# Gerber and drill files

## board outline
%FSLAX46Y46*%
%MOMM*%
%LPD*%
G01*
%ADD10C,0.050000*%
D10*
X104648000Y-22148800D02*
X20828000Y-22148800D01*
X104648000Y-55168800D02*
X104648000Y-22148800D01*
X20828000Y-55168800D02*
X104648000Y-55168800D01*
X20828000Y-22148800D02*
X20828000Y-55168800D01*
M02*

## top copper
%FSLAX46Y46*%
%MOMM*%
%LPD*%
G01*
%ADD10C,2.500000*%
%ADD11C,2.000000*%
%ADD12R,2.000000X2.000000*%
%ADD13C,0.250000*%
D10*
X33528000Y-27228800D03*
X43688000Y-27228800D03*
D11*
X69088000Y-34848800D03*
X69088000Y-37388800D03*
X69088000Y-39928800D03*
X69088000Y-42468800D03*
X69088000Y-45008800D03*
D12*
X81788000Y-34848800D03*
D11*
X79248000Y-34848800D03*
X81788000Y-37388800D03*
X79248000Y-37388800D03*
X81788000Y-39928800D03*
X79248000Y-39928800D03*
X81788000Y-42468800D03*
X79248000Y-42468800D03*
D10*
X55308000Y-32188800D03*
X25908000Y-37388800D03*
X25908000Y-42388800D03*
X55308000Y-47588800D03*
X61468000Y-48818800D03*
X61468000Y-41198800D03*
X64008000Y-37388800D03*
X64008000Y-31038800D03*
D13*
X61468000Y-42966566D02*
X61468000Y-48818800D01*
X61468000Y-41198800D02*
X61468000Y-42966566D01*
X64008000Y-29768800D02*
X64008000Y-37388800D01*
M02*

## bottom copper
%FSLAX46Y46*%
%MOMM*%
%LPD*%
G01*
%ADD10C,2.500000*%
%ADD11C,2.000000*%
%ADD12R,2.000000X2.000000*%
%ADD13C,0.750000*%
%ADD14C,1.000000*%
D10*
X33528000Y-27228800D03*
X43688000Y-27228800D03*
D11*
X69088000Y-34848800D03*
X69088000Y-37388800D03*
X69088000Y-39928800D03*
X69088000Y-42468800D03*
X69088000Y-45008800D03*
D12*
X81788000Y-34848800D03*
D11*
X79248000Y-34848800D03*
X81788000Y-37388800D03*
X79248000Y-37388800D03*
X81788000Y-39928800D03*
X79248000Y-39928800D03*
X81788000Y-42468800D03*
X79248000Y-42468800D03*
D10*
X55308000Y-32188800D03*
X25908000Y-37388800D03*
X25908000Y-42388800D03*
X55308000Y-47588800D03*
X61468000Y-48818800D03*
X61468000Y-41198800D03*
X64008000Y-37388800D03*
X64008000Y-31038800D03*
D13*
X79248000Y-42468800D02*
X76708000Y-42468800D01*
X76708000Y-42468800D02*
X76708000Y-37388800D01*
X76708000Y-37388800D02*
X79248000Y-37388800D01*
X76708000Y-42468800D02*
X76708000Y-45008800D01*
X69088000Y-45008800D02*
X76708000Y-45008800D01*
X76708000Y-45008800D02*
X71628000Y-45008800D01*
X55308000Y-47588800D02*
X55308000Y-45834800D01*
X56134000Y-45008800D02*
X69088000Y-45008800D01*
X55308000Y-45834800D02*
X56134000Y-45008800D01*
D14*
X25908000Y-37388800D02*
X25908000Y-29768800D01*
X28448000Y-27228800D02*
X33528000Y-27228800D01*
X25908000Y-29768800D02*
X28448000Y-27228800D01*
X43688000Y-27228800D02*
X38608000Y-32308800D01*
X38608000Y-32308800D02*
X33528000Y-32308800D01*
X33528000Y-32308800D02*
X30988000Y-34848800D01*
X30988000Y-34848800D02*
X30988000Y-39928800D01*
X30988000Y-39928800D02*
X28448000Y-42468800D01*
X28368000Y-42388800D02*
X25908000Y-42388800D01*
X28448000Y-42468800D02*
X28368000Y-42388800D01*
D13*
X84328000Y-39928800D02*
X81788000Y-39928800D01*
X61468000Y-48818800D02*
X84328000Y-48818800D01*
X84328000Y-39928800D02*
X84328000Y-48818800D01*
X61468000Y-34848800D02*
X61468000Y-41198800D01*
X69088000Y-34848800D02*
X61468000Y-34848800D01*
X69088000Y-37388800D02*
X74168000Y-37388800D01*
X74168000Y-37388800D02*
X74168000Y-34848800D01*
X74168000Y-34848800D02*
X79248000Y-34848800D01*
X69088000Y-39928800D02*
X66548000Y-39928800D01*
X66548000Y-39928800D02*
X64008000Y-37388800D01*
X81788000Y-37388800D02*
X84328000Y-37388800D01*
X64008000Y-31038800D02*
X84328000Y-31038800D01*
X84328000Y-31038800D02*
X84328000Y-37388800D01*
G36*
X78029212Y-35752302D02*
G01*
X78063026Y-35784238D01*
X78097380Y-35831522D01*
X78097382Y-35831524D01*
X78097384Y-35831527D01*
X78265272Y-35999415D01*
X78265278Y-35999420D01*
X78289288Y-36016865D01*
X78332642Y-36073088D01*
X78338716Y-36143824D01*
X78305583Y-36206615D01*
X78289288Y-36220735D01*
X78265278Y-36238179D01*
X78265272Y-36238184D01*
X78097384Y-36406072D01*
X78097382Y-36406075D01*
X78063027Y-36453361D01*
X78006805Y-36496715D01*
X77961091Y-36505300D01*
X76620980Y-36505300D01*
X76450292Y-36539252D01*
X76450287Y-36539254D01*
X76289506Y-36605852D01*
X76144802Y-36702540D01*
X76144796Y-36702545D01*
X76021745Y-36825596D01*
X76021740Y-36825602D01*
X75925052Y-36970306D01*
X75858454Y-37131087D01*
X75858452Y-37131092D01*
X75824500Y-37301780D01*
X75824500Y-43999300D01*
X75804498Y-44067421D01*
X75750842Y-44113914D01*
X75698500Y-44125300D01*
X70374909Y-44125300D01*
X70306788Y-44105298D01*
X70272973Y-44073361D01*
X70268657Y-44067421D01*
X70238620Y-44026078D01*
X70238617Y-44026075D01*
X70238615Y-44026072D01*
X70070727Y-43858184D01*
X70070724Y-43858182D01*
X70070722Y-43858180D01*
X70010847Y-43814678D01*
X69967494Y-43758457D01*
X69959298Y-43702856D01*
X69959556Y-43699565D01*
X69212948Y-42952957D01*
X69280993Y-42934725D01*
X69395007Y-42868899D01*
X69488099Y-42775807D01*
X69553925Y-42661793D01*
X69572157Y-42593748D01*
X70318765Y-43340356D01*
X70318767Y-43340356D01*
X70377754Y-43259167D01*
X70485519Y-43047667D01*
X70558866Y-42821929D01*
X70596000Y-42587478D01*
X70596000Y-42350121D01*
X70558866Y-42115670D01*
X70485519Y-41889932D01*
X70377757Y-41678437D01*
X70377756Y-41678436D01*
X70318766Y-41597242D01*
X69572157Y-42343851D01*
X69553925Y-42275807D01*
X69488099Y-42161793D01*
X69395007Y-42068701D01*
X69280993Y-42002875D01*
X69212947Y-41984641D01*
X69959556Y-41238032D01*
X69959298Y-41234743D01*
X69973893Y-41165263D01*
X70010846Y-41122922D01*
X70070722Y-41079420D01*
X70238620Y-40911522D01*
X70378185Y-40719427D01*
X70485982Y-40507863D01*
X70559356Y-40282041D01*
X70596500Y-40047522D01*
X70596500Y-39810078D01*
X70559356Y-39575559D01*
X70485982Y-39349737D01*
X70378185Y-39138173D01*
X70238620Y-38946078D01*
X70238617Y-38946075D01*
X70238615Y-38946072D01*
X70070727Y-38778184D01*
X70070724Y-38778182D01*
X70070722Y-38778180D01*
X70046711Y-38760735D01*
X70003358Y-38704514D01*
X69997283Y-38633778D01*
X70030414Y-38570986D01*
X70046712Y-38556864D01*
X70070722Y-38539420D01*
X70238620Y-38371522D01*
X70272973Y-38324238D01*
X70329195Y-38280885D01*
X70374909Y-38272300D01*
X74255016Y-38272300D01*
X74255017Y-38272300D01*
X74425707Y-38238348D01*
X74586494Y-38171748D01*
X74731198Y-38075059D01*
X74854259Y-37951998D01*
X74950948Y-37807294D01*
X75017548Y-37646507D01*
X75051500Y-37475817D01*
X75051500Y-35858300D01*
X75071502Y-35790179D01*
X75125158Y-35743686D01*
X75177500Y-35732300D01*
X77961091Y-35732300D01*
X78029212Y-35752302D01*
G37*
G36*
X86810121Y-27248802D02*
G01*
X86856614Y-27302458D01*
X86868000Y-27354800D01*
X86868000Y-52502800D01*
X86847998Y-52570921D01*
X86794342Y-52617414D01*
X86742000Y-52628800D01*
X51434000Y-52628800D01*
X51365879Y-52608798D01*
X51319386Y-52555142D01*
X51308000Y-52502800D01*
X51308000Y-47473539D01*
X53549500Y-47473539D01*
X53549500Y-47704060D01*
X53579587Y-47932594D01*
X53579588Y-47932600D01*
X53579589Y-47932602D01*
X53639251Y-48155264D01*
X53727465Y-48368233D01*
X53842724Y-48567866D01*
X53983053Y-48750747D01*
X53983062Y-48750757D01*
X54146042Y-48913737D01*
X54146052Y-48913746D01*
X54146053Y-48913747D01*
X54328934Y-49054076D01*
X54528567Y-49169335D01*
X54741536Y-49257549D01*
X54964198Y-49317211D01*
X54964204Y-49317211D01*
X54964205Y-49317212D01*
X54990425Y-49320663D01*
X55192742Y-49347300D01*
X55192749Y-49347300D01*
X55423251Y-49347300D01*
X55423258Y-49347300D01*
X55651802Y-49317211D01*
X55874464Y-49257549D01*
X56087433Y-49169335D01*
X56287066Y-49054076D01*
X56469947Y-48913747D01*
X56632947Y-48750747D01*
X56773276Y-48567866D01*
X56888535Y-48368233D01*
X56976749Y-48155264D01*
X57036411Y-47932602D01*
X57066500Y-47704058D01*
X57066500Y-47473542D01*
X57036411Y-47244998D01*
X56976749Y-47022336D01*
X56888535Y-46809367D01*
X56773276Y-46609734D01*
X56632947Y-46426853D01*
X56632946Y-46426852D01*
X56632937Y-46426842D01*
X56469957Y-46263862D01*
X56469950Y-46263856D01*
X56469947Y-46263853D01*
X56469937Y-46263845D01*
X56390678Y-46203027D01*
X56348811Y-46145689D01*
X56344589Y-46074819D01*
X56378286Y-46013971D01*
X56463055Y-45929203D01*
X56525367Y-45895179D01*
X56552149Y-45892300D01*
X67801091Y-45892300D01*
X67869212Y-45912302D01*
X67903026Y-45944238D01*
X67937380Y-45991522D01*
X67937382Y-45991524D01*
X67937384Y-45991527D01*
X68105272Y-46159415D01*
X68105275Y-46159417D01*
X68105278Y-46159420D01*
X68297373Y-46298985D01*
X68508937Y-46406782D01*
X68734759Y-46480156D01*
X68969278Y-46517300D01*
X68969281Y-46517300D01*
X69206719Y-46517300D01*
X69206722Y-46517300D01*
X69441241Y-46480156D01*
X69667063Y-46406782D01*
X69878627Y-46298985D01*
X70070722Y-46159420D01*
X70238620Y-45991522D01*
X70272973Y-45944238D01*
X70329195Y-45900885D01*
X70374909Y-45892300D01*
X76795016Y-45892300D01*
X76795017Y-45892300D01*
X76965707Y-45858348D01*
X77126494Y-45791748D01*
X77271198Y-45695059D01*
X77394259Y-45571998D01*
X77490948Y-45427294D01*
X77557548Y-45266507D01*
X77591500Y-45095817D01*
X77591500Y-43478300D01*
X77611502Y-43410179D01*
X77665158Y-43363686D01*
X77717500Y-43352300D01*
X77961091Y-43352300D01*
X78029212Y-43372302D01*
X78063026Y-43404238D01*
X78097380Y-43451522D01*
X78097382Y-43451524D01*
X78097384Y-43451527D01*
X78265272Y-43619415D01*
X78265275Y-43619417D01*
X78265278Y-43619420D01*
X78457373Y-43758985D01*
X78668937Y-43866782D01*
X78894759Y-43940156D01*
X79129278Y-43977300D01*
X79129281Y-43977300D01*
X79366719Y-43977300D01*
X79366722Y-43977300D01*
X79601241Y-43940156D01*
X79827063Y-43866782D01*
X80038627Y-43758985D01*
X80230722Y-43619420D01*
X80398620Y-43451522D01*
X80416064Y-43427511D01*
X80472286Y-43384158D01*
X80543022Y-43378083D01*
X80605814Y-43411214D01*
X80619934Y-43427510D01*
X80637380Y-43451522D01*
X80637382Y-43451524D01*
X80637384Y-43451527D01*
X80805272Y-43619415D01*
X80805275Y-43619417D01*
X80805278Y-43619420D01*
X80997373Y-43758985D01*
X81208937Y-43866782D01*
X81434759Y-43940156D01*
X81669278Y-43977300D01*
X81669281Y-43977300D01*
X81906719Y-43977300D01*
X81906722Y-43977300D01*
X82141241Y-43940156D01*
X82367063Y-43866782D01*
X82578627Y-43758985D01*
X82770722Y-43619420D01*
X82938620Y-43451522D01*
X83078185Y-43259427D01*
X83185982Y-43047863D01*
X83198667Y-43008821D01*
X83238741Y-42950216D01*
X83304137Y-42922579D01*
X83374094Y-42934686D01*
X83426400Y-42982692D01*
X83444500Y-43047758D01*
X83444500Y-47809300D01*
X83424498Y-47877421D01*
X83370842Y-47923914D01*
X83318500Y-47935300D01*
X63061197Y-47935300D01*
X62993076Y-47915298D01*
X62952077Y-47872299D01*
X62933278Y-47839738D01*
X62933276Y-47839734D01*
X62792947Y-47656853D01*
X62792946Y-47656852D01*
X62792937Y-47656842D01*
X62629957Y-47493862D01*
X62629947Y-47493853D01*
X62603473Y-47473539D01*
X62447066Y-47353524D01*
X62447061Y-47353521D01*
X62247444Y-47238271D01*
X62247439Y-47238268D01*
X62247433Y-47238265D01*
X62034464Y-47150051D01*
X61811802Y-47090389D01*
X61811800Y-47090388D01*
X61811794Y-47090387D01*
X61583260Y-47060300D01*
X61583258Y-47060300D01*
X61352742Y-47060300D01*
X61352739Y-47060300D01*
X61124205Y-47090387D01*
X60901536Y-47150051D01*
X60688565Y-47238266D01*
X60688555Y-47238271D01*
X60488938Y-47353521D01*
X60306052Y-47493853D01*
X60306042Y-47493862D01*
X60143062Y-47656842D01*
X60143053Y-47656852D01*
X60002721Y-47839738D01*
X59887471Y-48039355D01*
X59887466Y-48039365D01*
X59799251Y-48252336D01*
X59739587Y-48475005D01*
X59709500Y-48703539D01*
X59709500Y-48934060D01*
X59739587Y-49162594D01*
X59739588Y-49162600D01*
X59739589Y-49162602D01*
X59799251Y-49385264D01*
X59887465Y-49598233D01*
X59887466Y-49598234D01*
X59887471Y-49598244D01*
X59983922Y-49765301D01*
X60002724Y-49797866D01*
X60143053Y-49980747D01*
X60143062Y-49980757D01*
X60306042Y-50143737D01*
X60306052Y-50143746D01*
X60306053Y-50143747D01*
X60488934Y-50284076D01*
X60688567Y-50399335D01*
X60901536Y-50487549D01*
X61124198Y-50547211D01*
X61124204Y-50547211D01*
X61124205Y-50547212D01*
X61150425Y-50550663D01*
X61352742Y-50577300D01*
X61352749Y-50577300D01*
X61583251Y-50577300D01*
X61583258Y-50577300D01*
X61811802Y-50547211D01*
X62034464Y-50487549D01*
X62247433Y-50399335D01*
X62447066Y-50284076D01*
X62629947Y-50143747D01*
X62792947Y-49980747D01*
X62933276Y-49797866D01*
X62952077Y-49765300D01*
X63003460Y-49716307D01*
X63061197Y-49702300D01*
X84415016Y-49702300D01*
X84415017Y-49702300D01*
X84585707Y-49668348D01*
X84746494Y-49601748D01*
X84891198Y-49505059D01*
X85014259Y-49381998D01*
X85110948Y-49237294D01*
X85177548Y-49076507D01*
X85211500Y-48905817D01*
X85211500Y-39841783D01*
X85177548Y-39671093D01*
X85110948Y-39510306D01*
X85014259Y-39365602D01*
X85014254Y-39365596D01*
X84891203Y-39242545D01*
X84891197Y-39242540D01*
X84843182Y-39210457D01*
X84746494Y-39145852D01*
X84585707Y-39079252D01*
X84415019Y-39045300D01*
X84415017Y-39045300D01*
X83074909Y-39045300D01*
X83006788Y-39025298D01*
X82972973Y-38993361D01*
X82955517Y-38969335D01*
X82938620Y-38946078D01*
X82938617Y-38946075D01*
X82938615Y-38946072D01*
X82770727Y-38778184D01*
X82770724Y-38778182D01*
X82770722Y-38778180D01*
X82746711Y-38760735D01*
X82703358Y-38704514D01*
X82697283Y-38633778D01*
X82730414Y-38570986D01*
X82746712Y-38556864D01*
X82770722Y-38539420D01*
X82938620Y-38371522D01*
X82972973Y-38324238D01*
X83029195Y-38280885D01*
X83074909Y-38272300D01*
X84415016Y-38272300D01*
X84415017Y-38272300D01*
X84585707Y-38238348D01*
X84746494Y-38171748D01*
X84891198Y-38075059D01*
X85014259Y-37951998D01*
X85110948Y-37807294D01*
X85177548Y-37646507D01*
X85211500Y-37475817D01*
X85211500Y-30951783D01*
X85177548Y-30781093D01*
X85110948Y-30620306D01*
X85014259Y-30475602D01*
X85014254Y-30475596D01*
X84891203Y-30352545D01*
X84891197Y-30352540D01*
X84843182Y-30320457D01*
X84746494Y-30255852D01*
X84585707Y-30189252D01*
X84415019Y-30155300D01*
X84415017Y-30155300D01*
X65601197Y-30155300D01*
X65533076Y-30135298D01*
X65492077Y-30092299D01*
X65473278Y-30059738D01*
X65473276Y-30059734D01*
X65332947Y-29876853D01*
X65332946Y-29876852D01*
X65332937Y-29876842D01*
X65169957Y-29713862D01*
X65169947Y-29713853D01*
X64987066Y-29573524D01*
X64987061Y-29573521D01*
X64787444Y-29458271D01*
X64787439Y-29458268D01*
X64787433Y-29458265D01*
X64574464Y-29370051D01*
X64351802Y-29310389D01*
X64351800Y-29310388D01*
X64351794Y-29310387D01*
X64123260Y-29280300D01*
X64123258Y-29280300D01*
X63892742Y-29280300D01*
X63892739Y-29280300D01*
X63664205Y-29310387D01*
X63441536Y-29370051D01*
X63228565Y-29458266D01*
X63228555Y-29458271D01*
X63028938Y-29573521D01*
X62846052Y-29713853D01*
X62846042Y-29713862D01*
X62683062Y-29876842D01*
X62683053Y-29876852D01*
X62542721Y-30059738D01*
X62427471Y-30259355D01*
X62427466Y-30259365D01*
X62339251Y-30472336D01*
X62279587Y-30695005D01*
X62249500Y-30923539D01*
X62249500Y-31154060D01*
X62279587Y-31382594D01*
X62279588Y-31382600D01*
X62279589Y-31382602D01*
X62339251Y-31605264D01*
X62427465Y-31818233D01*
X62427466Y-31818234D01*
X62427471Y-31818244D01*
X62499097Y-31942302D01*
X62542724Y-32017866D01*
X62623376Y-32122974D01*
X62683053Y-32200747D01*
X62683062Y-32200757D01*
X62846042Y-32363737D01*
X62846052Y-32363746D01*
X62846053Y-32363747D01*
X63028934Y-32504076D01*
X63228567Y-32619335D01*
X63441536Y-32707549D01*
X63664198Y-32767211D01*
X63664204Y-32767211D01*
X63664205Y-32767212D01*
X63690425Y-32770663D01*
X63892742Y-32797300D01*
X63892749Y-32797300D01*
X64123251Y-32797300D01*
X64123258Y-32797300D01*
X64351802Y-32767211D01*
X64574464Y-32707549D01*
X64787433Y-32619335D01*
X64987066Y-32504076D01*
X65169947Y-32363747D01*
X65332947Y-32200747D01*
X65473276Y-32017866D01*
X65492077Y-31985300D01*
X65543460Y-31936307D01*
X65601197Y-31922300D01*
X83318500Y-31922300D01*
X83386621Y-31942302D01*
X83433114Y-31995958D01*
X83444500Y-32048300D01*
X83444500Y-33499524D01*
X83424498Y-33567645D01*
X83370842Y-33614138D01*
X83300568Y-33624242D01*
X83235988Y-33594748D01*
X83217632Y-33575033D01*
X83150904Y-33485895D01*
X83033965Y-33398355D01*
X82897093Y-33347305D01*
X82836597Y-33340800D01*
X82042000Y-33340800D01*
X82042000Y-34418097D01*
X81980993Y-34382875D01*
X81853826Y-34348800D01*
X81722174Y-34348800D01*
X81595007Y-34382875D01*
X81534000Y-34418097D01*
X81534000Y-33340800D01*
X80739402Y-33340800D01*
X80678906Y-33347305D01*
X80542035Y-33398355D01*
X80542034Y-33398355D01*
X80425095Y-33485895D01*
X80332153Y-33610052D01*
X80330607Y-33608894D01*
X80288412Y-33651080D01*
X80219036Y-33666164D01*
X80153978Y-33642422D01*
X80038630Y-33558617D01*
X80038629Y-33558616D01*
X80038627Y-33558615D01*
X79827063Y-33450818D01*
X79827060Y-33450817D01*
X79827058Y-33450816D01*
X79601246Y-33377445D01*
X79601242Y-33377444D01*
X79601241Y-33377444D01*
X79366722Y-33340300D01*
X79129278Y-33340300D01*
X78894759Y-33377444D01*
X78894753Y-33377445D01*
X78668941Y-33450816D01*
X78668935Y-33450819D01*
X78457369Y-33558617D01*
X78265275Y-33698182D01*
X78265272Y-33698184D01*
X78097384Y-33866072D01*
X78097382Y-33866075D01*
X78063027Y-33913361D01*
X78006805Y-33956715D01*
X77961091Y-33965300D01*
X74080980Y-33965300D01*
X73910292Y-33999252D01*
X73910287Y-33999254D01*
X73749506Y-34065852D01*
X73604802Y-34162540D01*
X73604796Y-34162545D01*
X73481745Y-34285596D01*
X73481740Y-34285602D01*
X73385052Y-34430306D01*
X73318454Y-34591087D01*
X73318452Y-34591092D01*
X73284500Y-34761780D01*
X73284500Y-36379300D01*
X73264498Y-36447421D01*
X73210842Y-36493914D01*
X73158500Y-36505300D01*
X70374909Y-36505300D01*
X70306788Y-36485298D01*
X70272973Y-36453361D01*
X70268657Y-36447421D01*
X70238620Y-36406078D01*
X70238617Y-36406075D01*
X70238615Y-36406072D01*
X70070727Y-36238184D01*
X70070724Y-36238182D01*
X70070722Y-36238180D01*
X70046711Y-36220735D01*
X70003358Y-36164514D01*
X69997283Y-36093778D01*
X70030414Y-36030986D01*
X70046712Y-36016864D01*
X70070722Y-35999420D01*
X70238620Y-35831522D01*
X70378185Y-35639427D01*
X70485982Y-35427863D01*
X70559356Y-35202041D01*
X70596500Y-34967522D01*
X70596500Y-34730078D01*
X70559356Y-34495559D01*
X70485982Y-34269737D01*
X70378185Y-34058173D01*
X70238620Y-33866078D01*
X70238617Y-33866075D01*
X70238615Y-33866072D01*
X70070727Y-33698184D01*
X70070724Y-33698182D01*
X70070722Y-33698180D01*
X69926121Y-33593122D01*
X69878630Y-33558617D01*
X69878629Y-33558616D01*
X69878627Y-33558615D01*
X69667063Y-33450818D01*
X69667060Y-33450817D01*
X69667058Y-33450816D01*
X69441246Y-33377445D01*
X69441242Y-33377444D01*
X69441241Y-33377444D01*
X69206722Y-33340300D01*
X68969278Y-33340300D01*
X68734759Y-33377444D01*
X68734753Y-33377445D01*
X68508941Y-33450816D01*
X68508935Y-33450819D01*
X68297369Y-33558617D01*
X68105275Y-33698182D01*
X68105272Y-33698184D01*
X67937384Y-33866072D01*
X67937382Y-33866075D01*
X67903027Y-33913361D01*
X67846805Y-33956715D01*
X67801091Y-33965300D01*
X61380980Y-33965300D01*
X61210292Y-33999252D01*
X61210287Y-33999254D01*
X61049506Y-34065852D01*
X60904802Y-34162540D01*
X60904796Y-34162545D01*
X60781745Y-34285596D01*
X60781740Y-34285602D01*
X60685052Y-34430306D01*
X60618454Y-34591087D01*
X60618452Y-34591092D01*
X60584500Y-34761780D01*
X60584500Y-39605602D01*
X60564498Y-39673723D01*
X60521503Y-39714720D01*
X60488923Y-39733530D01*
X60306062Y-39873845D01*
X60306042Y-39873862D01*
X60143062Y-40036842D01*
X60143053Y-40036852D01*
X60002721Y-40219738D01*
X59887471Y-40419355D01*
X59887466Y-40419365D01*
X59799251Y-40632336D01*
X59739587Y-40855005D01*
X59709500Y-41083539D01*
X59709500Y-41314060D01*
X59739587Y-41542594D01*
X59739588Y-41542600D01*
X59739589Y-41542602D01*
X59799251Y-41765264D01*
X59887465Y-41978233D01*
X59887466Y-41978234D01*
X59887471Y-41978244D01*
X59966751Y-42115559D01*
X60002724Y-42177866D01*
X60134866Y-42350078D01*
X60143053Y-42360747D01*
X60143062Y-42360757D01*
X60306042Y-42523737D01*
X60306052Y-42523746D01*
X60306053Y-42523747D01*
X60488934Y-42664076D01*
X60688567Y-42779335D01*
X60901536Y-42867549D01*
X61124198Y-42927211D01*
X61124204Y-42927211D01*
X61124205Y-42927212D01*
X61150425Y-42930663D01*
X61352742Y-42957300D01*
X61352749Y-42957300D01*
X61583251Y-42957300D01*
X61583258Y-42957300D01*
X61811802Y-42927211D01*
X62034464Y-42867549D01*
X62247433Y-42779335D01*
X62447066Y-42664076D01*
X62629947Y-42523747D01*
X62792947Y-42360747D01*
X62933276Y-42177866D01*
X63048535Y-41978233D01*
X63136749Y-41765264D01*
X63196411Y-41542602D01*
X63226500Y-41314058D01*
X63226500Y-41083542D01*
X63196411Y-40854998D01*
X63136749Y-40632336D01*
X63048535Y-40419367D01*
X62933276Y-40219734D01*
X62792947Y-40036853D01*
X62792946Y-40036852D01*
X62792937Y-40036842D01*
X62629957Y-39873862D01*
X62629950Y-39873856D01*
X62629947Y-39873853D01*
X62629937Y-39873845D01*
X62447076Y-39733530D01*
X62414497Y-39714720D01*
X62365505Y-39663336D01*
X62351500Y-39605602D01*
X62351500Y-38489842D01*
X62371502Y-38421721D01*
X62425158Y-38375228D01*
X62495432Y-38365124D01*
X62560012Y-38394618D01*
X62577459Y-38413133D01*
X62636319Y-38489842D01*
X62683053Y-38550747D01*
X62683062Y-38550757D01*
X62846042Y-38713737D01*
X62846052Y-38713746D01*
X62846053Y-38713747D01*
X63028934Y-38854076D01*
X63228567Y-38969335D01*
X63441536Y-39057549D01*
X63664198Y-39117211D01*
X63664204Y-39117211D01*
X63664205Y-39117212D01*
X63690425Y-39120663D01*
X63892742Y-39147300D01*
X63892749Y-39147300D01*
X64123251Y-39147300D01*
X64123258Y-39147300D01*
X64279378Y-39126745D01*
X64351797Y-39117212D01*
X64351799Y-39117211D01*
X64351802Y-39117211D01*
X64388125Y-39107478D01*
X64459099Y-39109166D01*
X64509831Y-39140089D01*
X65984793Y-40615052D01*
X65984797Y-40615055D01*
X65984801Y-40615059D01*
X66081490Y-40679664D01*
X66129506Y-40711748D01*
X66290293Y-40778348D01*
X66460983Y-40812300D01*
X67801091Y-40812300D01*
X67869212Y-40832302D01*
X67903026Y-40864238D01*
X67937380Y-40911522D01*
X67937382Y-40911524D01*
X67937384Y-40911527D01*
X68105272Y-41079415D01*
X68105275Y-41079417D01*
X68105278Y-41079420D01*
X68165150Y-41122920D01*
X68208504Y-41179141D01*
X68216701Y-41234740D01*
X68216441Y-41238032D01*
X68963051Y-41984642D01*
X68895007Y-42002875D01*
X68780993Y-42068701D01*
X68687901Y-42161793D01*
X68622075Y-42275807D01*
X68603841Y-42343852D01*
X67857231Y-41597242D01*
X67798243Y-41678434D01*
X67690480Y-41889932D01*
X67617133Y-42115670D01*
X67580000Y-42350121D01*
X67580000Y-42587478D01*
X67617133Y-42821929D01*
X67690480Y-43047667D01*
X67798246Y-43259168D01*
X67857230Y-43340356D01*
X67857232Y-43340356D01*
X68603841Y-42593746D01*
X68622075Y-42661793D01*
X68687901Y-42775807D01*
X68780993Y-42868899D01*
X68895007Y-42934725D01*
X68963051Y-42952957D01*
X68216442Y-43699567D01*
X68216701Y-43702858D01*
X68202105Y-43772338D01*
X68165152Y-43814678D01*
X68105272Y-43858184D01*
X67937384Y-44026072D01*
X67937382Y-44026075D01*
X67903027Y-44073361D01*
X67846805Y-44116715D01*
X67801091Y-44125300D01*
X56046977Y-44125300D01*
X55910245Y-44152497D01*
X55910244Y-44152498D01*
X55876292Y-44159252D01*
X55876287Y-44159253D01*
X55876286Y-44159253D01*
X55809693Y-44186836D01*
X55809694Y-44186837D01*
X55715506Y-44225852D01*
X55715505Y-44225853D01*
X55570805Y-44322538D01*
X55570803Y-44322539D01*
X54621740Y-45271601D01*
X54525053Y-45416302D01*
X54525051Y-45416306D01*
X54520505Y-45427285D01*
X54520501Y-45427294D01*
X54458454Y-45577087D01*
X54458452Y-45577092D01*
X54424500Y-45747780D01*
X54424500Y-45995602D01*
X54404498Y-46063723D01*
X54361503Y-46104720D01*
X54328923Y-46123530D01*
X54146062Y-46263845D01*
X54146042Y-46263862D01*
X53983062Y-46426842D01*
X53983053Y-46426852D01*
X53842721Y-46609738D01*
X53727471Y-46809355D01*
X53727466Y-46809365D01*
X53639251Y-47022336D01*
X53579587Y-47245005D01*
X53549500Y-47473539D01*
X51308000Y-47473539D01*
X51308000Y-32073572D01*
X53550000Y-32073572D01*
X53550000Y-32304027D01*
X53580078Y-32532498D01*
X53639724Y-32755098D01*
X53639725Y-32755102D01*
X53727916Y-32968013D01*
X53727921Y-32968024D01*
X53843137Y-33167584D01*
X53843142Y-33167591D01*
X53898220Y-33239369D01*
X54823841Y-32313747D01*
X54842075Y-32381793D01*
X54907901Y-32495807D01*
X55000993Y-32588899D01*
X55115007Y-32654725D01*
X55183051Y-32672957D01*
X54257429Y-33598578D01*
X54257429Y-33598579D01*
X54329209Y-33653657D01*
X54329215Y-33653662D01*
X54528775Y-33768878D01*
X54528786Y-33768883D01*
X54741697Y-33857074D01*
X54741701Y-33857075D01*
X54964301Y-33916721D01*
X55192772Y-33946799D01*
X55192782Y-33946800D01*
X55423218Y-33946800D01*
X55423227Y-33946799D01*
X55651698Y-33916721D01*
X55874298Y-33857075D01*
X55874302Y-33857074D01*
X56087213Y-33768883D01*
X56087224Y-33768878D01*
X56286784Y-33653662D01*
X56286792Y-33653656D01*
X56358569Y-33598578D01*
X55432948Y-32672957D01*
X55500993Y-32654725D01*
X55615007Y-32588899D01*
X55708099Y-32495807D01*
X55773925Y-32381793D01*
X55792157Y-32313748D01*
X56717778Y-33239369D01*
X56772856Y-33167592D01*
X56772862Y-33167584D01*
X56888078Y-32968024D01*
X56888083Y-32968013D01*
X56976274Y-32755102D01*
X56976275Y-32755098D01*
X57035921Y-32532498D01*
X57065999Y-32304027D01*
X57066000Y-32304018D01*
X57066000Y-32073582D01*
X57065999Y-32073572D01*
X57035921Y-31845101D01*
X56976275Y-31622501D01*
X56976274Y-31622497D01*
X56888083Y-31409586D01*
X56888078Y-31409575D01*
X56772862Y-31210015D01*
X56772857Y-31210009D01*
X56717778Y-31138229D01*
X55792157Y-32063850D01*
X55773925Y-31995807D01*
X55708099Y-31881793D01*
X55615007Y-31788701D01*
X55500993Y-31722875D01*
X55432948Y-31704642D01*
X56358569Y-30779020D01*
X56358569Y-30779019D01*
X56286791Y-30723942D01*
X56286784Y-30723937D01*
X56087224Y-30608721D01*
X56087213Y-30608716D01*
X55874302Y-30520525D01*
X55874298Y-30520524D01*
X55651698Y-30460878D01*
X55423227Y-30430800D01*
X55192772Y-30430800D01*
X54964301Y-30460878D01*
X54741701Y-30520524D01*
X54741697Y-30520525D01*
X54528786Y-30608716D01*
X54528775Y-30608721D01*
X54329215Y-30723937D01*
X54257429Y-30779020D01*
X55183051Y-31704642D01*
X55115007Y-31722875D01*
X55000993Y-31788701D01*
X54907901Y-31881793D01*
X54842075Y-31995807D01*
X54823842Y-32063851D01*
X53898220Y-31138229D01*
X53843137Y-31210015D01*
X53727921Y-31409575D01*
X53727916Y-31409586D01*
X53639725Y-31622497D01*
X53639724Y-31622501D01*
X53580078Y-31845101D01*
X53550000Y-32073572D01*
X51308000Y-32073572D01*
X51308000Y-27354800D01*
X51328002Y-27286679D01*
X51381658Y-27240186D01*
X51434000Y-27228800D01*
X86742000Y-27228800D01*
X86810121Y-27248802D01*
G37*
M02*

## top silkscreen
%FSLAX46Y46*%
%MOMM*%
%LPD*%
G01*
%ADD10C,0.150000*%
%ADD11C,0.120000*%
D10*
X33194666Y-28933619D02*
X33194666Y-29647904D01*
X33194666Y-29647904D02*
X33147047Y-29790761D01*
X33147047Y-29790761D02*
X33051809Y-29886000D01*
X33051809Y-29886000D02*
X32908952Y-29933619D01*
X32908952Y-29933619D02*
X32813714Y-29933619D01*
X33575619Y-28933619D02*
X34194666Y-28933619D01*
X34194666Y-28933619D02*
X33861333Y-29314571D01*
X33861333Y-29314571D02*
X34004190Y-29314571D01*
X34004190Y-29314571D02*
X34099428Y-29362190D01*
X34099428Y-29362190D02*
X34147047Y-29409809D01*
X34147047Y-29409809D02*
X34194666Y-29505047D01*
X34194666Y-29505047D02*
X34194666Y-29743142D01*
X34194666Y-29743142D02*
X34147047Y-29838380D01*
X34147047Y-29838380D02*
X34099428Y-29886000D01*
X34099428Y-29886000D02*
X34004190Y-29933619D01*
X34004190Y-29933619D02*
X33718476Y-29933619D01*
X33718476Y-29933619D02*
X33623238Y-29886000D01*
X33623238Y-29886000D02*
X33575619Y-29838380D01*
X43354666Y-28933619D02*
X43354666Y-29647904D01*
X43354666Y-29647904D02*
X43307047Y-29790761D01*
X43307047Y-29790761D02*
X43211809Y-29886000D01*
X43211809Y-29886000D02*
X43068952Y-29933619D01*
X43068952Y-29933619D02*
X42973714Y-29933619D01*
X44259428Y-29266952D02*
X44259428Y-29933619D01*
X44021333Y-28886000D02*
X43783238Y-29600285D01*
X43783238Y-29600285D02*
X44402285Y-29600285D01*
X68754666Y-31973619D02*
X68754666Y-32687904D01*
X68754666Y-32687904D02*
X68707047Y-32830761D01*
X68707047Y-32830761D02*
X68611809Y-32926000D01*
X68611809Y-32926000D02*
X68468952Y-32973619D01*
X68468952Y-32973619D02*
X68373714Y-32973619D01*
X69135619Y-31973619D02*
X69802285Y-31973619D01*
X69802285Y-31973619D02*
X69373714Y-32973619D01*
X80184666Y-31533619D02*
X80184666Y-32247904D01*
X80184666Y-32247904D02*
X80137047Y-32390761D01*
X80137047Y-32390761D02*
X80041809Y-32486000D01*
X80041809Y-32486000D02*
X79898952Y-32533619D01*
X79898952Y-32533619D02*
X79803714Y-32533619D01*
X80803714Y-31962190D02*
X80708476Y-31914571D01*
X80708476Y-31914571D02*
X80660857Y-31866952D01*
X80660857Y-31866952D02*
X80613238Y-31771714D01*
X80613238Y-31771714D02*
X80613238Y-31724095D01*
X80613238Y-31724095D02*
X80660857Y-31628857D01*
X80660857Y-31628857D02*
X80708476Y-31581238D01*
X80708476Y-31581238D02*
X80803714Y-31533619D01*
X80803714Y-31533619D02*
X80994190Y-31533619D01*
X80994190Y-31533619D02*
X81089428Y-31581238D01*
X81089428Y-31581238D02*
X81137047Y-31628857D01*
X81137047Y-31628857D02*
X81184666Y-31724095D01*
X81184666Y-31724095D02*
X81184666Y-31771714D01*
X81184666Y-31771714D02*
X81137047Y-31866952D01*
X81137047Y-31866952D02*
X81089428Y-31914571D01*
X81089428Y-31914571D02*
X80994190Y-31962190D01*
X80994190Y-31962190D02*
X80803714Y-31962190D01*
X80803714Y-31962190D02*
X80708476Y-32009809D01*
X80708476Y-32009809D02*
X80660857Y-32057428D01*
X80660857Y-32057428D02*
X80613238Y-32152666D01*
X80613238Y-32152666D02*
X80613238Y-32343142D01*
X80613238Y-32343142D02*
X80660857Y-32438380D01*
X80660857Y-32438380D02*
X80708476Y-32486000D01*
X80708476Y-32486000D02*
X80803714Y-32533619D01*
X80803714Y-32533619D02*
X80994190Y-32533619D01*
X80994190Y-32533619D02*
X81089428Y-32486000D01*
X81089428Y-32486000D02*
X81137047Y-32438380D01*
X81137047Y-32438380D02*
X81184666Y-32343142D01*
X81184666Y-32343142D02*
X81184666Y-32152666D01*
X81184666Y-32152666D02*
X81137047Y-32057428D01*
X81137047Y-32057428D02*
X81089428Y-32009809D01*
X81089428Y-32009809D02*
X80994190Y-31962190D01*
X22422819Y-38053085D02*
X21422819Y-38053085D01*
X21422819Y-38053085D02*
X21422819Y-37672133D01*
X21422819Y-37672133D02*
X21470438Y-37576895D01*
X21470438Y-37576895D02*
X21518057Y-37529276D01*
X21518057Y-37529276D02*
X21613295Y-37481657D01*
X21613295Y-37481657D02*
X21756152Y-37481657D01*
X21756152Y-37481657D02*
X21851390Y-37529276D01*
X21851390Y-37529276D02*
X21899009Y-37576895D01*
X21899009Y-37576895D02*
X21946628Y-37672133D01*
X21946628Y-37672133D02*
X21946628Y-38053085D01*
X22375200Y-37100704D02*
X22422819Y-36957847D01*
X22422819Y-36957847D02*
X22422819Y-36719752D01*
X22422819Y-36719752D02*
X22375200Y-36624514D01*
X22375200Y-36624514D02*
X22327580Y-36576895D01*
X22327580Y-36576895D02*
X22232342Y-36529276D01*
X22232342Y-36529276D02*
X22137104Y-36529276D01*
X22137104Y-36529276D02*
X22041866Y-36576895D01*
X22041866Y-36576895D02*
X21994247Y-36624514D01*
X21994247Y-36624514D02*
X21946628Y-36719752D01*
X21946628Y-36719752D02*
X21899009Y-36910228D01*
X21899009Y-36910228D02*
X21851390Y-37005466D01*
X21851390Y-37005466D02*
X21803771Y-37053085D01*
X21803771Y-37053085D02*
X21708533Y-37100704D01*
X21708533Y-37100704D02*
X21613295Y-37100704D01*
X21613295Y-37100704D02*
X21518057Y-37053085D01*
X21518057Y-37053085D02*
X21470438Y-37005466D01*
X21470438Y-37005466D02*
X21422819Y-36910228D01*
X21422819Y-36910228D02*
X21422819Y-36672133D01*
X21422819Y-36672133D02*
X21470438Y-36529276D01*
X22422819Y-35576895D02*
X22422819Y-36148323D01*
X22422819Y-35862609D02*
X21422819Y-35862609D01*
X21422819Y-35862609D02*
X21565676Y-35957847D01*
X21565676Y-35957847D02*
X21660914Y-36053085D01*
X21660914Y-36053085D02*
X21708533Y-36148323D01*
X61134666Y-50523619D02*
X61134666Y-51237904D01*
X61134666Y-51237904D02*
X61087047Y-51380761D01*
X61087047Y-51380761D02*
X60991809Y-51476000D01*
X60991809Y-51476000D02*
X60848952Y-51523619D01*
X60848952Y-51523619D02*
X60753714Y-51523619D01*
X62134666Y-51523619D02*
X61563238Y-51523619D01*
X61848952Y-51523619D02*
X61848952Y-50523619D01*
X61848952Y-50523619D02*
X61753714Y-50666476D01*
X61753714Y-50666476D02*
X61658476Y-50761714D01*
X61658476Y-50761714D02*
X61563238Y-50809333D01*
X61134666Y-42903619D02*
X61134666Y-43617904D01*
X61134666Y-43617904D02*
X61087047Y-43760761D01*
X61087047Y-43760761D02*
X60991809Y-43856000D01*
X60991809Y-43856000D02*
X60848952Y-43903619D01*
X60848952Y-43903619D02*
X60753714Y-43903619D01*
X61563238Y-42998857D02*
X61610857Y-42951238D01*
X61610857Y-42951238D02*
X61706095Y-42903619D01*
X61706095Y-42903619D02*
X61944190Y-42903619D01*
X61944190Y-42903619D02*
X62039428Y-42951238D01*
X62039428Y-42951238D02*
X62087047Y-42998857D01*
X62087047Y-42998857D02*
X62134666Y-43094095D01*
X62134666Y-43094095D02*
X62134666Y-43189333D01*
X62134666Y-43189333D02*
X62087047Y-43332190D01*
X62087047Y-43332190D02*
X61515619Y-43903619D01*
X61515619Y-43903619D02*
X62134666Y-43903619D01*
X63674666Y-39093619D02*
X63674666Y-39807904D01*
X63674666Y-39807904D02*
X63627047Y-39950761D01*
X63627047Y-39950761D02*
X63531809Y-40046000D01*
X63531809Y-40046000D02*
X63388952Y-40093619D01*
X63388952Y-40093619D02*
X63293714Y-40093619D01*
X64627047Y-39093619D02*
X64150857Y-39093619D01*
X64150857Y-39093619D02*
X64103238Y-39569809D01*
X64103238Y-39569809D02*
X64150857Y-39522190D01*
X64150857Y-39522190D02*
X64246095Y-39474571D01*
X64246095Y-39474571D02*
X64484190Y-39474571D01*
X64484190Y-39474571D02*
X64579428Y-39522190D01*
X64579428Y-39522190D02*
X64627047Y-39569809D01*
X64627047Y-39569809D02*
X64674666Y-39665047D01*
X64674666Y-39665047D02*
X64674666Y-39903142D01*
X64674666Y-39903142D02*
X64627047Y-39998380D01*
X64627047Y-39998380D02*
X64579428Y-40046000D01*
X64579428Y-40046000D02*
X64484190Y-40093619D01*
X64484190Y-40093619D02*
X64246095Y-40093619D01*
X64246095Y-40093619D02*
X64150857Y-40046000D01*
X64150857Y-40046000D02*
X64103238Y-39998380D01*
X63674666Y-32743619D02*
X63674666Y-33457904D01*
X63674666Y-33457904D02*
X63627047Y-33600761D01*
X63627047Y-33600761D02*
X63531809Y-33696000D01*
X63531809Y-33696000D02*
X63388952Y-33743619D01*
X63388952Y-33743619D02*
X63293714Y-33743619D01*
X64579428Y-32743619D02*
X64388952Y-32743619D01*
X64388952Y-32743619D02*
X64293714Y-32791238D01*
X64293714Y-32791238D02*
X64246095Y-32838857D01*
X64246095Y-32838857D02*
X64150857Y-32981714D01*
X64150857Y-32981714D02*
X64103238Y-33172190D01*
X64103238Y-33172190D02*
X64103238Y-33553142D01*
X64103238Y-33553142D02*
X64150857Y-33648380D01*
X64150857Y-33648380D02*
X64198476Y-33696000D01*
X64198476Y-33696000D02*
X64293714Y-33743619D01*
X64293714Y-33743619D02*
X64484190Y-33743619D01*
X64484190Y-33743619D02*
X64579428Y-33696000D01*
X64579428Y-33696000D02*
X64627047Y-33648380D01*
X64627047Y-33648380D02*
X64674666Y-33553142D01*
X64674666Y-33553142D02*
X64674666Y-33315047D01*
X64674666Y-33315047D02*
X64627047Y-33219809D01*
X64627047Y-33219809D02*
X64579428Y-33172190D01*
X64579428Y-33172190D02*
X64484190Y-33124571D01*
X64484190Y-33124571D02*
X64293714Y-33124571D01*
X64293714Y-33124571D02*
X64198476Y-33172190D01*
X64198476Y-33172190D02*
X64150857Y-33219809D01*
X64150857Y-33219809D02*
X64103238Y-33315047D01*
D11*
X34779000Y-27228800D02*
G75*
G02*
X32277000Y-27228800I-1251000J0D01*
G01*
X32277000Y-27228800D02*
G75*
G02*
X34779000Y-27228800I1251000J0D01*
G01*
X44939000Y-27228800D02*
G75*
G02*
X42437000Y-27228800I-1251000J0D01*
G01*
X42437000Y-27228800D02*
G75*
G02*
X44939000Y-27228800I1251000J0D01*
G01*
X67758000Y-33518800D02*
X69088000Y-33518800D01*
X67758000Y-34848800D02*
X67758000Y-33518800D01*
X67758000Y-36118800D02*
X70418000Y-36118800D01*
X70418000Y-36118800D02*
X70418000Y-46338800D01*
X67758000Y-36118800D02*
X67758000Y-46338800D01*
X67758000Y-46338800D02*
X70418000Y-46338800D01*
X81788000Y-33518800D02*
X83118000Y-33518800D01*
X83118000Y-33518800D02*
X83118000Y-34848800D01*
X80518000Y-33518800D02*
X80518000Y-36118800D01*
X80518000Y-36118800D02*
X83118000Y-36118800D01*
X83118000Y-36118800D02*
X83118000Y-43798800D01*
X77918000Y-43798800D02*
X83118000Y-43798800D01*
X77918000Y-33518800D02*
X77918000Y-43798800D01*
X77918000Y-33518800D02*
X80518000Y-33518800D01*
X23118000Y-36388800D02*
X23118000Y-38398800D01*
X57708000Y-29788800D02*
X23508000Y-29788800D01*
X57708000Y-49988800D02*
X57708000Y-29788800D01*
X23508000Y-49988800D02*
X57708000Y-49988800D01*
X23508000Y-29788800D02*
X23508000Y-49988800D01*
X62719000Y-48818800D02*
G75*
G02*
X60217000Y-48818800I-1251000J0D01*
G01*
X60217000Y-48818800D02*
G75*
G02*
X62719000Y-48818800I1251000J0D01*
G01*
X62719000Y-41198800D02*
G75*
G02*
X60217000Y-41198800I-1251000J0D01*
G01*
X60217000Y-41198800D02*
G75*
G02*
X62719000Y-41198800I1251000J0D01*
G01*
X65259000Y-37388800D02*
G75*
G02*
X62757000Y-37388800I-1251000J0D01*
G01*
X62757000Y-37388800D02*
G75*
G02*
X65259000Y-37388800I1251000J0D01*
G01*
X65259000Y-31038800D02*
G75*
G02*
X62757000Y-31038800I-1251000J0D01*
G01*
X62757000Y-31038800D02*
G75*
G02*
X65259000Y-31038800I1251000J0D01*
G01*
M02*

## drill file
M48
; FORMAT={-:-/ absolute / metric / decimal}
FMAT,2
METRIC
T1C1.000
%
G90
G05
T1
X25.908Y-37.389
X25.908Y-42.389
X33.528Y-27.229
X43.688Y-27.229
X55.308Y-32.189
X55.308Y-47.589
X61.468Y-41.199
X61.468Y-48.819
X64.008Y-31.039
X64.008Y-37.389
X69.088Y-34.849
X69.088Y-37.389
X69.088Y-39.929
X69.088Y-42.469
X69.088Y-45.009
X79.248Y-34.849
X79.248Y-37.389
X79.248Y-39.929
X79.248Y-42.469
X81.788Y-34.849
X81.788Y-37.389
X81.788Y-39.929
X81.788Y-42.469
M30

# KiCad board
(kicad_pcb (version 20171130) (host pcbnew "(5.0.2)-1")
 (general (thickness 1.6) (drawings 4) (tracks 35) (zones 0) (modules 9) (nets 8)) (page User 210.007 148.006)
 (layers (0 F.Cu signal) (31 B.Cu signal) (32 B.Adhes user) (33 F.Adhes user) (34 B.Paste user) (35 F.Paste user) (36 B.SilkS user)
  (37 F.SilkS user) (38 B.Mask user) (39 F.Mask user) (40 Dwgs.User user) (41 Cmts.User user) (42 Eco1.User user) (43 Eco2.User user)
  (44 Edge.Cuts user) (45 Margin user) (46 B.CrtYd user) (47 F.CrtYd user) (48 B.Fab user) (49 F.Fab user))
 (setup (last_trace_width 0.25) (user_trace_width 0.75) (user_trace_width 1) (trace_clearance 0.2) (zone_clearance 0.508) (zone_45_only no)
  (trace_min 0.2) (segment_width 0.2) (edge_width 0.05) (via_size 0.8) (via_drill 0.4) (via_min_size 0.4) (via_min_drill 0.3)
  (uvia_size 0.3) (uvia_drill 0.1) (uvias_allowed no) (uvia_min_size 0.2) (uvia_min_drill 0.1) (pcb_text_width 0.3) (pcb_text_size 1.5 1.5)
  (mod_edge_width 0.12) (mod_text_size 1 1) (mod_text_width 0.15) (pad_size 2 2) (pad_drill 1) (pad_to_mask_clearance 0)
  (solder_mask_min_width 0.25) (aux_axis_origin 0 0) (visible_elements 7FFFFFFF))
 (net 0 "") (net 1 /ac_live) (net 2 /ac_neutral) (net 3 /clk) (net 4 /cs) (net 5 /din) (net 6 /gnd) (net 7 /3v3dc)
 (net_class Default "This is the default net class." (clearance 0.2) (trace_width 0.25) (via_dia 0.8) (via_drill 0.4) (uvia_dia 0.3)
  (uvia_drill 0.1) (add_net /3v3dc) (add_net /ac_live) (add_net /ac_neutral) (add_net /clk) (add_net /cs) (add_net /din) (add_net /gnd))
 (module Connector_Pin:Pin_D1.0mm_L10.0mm (layer F.Cu) (at 33.528 27.2288)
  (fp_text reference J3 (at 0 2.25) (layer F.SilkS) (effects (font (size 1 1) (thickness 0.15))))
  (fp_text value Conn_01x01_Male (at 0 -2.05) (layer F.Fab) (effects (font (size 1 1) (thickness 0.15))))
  (fp_circle (center 0 0) (end 1.25 0.05) (layer F.SilkS) (width 0.12))
  (pad 1 thru_hole circle (at 0 0) (size 2.5 2.5) (drill 1) (layers *.Cu *.Mask) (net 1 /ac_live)))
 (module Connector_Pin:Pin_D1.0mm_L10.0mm (layer F.Cu) (at 43.688 27.2288)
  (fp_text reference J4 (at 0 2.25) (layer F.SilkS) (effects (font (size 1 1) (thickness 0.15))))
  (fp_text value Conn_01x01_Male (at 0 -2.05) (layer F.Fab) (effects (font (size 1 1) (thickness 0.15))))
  (fp_circle (center 0 0) (end 1.25 0.05) (layer F.SilkS) (width 0.12))
  (pad 1 thru_hole circle (at 0 0) (size 2.5 2.5) (drill 1) (layers *.Cu *.Mask) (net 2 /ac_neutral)))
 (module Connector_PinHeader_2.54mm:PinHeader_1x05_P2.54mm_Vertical (layer F.Cu) (at 69.088 34.8488)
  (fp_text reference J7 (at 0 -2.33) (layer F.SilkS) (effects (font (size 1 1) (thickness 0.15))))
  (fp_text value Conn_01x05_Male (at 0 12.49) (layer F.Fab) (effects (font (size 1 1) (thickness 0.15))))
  (fp_line (start -1.33 -1.33) (end 0 -1.33) (layer F.SilkS) (width 0.12))
  (fp_line (start -1.33 0) (end -1.33 -1.33) (layer F.SilkS) (width 0.12))
  (fp_line (start -1.33 1.27) (end 1.33 1.27) (layer F.SilkS) (width 0.12))
  (fp_line (start 1.33 1.27) (end 1.33 11.49) (layer F.SilkS) (width 0.12))
  (fp_line (start -1.33 1.27) (end -1.33 11.49) (layer F.SilkS) (width 0.12))
  (fp_line (start -1.33 11.49) (end 1.33 11.49) (layer F.SilkS) (width 0.12))
  (pad 1 thru_hole circle (at 0 0) (size 2 2) (drill 1) (layers *.Cu *.Mask) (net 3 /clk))
  (pad 2 thru_hole circle (at 0 2.54) (size 2 2) (drill 1) (layers *.Cu *.Mask) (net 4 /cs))
  (pad 3 thru_hole circle (at 0 5.08) (size 2 2) (drill 1) (layers *.Cu *.Mask) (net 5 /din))
  (pad 4 thru_hole circle (at 0 7.62) (size 2 2) (drill 1) (layers *.Cu *.Mask) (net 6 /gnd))
  (pad 5 thru_hole circle (at 0 10.16) (size 2 2) (drill 1) (layers *.Cu *.Mask) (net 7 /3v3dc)))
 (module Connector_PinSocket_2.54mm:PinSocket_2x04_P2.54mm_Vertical (layer F.Cu) (at 81.788 34.8488)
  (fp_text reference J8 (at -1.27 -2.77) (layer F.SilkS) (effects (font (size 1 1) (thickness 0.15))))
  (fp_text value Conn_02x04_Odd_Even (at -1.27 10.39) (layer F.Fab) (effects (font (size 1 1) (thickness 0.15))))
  (fp_line (start 0 -1.33) (end 1.33 -1.33) (layer F.SilkS) (width 0.12))
  (fp_line (start 1.33 -1.33) (end 1.33 0) (layer F.SilkS) (width 0.12))
  (fp_line (start -1.27 -1.33) (end -1.27 1.27) (layer F.SilkS) (width 0.12))
  (fp_line (start -1.27 1.27) (end 1.33 1.27) (layer F.SilkS) (width 0.12))
  (fp_line (start 1.33 1.27) (end 1.33 8.95) (layer F.SilkS) (width 0.12))
  (fp_line (start -3.87 8.95) (end 1.33 8.95) (layer F.SilkS) (width 0.12))
  (fp_line (start -3.87 -1.33) (end -3.87 8.95) (layer F.SilkS) (width 0.12))
  (fp_line (start -3.87 -1.33) (end -1.27 -1.33) (layer F.SilkS) (width 0.12))
  (pad 1 thru_hole rect (at 0 0) (size 2 2) (drill 1) (layers *.Cu *.Mask) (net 6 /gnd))
  (pad 2 thru_hole circle (at -2.54 0) (size 2 2) (drill 1) (layers *.Cu *.Mask) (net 4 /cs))
  (pad 3 thru_hole circle (at 0 2.54) (size 2 2) (drill 1) (layers *.Cu *.Mask) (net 5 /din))
  (pad 4 thru_hole circle (at -2.54 2.54) (size 2 2) (drill 1) (layers *.Cu *.Mask) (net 7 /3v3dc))
  (pad 5 thru_hole circle (at 0 5.08) (size 2 2) (drill 1) (layers *.Cu *.Mask) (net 3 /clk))
  (pad 6 thru_hole circle (at -2.54 5.08) (size 2 2) (drill 1) (layers *.Cu *.Mask))
  (pad 7 thru_hole circle (at 0 7.62) (size 2 2) (drill 1) (layers *.Cu *.Mask))
  (pad 8 thru_hole circle (at -2.54 7.62) (size 2 2) (drill 1) (layers *.Cu *.Mask) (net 7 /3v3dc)))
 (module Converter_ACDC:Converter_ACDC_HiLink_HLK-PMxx (layer F.Cu) (at 25.908 37.3888)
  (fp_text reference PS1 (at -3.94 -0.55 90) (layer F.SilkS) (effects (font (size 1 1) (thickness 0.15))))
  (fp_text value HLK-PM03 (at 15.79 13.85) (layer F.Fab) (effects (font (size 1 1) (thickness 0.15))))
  (fp_line (start -2.79 -1) (end -2.79 1.01) (layer F.SilkS) (width 0.12))
  (fp_line (start 31.8 -7.6) (end -2.4 -7.6) (layer F.SilkS) (width 0.12))
  (fp_line (start 31.8 12.6) (end 31.8 -7.6) (layer F.SilkS) (width 0.12))
  (fp_line (start -2.4 12.6) (end 31.8 12.6) (layer F.SilkS) (width 0.12))
  (fp_line (start -2.4 -7.6) (end -2.4 12.6) (layer F.SilkS) (width 0.12))
  (pad 3 thru_hole circle (at 29.4 -5.2) (size 2.5 2.5) (drill 1) (layers *.Cu *.Mask) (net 6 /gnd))
  (pad 1 thru_hole circle (at 0 0) (size 2.5 2.5) (drill 1) (layers *.Cu *.Mask) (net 1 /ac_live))
  (pad 2 thru_hole circle (at 0 5) (size 2.5 2.5) (drill 1) (layers *.Cu *.Mask) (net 2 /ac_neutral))
  (pad 4 thru_hole circle (at 29.4 10.2) (size 2.5 2.5) (drill 1) (layers *.Cu *.Mask) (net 7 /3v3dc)))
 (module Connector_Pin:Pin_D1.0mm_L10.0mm (layer F.Cu) (at 61.468 48.8188)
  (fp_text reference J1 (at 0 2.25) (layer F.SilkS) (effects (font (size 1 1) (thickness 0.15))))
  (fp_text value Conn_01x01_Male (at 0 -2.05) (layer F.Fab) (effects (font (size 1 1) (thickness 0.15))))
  (fp_circle (center 0 0) (end 1.25 0.05) (layer F.SilkS) (width 0.12))
  (pad 1 thru_hole circle (at 0 0) (size 2.5 2.5) (drill 1) (layers *.Cu *.Mask) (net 3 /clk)))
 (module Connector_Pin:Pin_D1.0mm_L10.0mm (layer F.Cu) (at 61.468 41.1988)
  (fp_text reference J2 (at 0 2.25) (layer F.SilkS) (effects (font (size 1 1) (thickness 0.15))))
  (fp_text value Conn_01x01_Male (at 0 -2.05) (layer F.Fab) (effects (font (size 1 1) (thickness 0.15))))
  (fp_circle (center 0 0) (end 1.25 0.05) (layer F.SilkS) (width 0.12))
  (pad 1 thru_hole circle (at 0 0) (size 2.5 2.5) (drill 1) (layers *.Cu *.Mask) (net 3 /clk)))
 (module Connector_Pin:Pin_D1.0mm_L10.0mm (layer F.Cu) (at 64.008 37.3888)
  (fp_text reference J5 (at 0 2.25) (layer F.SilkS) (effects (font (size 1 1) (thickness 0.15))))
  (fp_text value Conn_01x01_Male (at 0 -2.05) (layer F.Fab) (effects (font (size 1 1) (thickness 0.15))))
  (fp_circle (center 0 0) (end 1.25 0.05) (layer F.SilkS) (width 0.12))
  (pad 1 thru_hole circle (at 0 0) (size 2.5 2.5) (drill 1) (layers *.Cu *.Mask) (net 5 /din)))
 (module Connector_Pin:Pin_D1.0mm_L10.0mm (layer F.Cu) (at 64.008 31.0388)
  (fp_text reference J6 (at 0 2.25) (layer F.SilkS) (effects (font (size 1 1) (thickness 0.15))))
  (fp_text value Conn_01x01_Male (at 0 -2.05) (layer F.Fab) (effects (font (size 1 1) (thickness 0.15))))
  (fp_circle (center 0 0) (end 1.25 0.05) (layer F.SilkS) (width 0.12))
  (pad 1 thru_hole circle (at 0 0) (size 2.5 2.5) (drill 1) (layers *.Cu *.Mask) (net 5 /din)))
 (gr_line (start 104.648 22.1488) (end 20.828 22.1488) (layer Edge.Cuts) (width 0.05))
 (gr_line (start 104.648 55.1688) (end 104.648 22.1488) (layer Edge.Cuts) (width 0.05))
 (gr_line (start 20.828 55.1688) (end 104.648 55.1688) (layer Edge.Cuts) (width 0.05))
 (gr_line (start 20.828 22.1488) (end 20.828 55.1688) (layer Edge.Cuts) (width 0.05))
 (segment (start 79.248 42.4688) (end 76.708 42.4688) (width 0.75) (layer B.Cu) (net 7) (status 10))
 (segment (start 76.708 42.4688) (end 76.708 37.3888) (width 0.75) (layer B.Cu) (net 7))
 (segment (start 76.708 37.3888) (end 79.248 37.3888) (width 0.75) (layer B.Cu) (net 7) (status 20))
 (segment (start 76.708 42.4688) (end 76.708 45.0088) (width 0.75) (layer B.Cu) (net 7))
 (segment (start 69.088 45.0088) (end 76.708 45.0088) (width 0.75) (layer B.Cu) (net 7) (status 10))
 (segment (start 76.708 45.0088) (end 71.628 45.0088) (width 0.75) (layer B.Cu) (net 7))
 (segment (start 55.308 47.5888) (end 55.308 45.8348) (width 0.75) (layer B.Cu) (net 7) (status 10))
 (segment (start 56.134 45.0088) (end 69.088 45.0088) (width 0.75) (layer B.Cu) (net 7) (status 20))
 (segment (start 55.308 45.8348) (end 56.134 45.0088) (width 0.75) (layer B.Cu) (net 7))
 (segment (start 25.908 37.3888) (end 25.908 29.7688) (width 1) (layer B.Cu) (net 1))
 (segment (start 28.448 27.2288) (end 33.528 27.2288) (width 1) (layer B.Cu) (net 1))
 (segment (start 25.908 29.7688) (end 28.448 27.2288) (width 1) (layer B.Cu) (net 1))
 (segment (start 43.688 27.2288) (end 38.608 32.3088) (width 1) (layer B.Cu) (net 2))
 (segment (start 38.608 32.3088) (end 33.528 32.3088) (width 1) (layer B.Cu) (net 2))
 (segment (start 33.528 32.3088) (end 30.988 34.8488) (width 1) (layer B.Cu) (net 2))
 (segment (start 30.988 34.8488) (end 30.988 39.9288) (width 1) (layer B.Cu) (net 2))
 (segment (start 30.988 39.9288) (end 28.448 42.4688) (width 1) (layer B.Cu) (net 2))
 (segment (start 28.368 42.3888) (end 25.908 42.3888) (width 1) (layer B.Cu) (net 2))
 (segment (start 28.448 42.4688) (end 28.368 42.3888) (width 1) (layer B.Cu) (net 2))
 (segment (start 84.328 39.9288) (end 81.788 39.9288) (width 0.75) (layer B.Cu) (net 3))
 (segment (start 61.468 48.8188) (end 84.328 48.8188) (width 0.75) (layer B.Cu) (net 3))
 (segment (start 84.328 39.9288) (end 84.328 48.8188) (width 0.75) (layer B.Cu) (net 3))
 (segment (start 61.468 42.966566) (end 61.468 48.8188) (width 0.25) (layer F.Cu) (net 3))
 (segment (start 61.468 41.1988) (end 61.468 42.966566) (width 0.25) (layer F.Cu) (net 3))
 (segment (start 61.468 34.8488) (end 61.468 41.1988) (width 0.75) (layer B.Cu) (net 3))
 (segment (start 69.088 34.8488) (end 61.468 34.8488) (width 0.75) (layer B.Cu) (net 3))
 (segment (start 69.088 37.3888) (end 74.168 37.3888) (width 0.75) (layer B.Cu) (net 4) (status 10))
 (segment (start 74.168 37.3888) (end 74.168 34.8488) (width 0.75) (layer B.Cu) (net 4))
 (segment (start 74.168 34.8488) (end 79.248 34.8488) (width 0.75) (layer B.Cu) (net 4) (status 20))
 (segment (start 69.088 39.9288) (end 66.548 39.9288) (width 0.75) (layer B.Cu) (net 5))
 (segment (start 66.548 39.9288) (end 64.008 37.3888) (width 0.75) (layer B.Cu) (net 5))
 (segment (start 64.008 29.7688) (end 64.008 37.3888) (width 0.25) (layer F.Cu) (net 5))
 (segment (start 81.788 37.3888) (end 84.328 37.3888) (width 0.75) (layer B.Cu) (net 5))
 (segment (start 64.008 31.0388) (end 84.328 31.0388) (width 0.75) (layer B.Cu) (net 5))
 (segment (start 84.328 31.0388) (end 84.328 37.3888) (width 0.75) (layer B.Cu) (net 5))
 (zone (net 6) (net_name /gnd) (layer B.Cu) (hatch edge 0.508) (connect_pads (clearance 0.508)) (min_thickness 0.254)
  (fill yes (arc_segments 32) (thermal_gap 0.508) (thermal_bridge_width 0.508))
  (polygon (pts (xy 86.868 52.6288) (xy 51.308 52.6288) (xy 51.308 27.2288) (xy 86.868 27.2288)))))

